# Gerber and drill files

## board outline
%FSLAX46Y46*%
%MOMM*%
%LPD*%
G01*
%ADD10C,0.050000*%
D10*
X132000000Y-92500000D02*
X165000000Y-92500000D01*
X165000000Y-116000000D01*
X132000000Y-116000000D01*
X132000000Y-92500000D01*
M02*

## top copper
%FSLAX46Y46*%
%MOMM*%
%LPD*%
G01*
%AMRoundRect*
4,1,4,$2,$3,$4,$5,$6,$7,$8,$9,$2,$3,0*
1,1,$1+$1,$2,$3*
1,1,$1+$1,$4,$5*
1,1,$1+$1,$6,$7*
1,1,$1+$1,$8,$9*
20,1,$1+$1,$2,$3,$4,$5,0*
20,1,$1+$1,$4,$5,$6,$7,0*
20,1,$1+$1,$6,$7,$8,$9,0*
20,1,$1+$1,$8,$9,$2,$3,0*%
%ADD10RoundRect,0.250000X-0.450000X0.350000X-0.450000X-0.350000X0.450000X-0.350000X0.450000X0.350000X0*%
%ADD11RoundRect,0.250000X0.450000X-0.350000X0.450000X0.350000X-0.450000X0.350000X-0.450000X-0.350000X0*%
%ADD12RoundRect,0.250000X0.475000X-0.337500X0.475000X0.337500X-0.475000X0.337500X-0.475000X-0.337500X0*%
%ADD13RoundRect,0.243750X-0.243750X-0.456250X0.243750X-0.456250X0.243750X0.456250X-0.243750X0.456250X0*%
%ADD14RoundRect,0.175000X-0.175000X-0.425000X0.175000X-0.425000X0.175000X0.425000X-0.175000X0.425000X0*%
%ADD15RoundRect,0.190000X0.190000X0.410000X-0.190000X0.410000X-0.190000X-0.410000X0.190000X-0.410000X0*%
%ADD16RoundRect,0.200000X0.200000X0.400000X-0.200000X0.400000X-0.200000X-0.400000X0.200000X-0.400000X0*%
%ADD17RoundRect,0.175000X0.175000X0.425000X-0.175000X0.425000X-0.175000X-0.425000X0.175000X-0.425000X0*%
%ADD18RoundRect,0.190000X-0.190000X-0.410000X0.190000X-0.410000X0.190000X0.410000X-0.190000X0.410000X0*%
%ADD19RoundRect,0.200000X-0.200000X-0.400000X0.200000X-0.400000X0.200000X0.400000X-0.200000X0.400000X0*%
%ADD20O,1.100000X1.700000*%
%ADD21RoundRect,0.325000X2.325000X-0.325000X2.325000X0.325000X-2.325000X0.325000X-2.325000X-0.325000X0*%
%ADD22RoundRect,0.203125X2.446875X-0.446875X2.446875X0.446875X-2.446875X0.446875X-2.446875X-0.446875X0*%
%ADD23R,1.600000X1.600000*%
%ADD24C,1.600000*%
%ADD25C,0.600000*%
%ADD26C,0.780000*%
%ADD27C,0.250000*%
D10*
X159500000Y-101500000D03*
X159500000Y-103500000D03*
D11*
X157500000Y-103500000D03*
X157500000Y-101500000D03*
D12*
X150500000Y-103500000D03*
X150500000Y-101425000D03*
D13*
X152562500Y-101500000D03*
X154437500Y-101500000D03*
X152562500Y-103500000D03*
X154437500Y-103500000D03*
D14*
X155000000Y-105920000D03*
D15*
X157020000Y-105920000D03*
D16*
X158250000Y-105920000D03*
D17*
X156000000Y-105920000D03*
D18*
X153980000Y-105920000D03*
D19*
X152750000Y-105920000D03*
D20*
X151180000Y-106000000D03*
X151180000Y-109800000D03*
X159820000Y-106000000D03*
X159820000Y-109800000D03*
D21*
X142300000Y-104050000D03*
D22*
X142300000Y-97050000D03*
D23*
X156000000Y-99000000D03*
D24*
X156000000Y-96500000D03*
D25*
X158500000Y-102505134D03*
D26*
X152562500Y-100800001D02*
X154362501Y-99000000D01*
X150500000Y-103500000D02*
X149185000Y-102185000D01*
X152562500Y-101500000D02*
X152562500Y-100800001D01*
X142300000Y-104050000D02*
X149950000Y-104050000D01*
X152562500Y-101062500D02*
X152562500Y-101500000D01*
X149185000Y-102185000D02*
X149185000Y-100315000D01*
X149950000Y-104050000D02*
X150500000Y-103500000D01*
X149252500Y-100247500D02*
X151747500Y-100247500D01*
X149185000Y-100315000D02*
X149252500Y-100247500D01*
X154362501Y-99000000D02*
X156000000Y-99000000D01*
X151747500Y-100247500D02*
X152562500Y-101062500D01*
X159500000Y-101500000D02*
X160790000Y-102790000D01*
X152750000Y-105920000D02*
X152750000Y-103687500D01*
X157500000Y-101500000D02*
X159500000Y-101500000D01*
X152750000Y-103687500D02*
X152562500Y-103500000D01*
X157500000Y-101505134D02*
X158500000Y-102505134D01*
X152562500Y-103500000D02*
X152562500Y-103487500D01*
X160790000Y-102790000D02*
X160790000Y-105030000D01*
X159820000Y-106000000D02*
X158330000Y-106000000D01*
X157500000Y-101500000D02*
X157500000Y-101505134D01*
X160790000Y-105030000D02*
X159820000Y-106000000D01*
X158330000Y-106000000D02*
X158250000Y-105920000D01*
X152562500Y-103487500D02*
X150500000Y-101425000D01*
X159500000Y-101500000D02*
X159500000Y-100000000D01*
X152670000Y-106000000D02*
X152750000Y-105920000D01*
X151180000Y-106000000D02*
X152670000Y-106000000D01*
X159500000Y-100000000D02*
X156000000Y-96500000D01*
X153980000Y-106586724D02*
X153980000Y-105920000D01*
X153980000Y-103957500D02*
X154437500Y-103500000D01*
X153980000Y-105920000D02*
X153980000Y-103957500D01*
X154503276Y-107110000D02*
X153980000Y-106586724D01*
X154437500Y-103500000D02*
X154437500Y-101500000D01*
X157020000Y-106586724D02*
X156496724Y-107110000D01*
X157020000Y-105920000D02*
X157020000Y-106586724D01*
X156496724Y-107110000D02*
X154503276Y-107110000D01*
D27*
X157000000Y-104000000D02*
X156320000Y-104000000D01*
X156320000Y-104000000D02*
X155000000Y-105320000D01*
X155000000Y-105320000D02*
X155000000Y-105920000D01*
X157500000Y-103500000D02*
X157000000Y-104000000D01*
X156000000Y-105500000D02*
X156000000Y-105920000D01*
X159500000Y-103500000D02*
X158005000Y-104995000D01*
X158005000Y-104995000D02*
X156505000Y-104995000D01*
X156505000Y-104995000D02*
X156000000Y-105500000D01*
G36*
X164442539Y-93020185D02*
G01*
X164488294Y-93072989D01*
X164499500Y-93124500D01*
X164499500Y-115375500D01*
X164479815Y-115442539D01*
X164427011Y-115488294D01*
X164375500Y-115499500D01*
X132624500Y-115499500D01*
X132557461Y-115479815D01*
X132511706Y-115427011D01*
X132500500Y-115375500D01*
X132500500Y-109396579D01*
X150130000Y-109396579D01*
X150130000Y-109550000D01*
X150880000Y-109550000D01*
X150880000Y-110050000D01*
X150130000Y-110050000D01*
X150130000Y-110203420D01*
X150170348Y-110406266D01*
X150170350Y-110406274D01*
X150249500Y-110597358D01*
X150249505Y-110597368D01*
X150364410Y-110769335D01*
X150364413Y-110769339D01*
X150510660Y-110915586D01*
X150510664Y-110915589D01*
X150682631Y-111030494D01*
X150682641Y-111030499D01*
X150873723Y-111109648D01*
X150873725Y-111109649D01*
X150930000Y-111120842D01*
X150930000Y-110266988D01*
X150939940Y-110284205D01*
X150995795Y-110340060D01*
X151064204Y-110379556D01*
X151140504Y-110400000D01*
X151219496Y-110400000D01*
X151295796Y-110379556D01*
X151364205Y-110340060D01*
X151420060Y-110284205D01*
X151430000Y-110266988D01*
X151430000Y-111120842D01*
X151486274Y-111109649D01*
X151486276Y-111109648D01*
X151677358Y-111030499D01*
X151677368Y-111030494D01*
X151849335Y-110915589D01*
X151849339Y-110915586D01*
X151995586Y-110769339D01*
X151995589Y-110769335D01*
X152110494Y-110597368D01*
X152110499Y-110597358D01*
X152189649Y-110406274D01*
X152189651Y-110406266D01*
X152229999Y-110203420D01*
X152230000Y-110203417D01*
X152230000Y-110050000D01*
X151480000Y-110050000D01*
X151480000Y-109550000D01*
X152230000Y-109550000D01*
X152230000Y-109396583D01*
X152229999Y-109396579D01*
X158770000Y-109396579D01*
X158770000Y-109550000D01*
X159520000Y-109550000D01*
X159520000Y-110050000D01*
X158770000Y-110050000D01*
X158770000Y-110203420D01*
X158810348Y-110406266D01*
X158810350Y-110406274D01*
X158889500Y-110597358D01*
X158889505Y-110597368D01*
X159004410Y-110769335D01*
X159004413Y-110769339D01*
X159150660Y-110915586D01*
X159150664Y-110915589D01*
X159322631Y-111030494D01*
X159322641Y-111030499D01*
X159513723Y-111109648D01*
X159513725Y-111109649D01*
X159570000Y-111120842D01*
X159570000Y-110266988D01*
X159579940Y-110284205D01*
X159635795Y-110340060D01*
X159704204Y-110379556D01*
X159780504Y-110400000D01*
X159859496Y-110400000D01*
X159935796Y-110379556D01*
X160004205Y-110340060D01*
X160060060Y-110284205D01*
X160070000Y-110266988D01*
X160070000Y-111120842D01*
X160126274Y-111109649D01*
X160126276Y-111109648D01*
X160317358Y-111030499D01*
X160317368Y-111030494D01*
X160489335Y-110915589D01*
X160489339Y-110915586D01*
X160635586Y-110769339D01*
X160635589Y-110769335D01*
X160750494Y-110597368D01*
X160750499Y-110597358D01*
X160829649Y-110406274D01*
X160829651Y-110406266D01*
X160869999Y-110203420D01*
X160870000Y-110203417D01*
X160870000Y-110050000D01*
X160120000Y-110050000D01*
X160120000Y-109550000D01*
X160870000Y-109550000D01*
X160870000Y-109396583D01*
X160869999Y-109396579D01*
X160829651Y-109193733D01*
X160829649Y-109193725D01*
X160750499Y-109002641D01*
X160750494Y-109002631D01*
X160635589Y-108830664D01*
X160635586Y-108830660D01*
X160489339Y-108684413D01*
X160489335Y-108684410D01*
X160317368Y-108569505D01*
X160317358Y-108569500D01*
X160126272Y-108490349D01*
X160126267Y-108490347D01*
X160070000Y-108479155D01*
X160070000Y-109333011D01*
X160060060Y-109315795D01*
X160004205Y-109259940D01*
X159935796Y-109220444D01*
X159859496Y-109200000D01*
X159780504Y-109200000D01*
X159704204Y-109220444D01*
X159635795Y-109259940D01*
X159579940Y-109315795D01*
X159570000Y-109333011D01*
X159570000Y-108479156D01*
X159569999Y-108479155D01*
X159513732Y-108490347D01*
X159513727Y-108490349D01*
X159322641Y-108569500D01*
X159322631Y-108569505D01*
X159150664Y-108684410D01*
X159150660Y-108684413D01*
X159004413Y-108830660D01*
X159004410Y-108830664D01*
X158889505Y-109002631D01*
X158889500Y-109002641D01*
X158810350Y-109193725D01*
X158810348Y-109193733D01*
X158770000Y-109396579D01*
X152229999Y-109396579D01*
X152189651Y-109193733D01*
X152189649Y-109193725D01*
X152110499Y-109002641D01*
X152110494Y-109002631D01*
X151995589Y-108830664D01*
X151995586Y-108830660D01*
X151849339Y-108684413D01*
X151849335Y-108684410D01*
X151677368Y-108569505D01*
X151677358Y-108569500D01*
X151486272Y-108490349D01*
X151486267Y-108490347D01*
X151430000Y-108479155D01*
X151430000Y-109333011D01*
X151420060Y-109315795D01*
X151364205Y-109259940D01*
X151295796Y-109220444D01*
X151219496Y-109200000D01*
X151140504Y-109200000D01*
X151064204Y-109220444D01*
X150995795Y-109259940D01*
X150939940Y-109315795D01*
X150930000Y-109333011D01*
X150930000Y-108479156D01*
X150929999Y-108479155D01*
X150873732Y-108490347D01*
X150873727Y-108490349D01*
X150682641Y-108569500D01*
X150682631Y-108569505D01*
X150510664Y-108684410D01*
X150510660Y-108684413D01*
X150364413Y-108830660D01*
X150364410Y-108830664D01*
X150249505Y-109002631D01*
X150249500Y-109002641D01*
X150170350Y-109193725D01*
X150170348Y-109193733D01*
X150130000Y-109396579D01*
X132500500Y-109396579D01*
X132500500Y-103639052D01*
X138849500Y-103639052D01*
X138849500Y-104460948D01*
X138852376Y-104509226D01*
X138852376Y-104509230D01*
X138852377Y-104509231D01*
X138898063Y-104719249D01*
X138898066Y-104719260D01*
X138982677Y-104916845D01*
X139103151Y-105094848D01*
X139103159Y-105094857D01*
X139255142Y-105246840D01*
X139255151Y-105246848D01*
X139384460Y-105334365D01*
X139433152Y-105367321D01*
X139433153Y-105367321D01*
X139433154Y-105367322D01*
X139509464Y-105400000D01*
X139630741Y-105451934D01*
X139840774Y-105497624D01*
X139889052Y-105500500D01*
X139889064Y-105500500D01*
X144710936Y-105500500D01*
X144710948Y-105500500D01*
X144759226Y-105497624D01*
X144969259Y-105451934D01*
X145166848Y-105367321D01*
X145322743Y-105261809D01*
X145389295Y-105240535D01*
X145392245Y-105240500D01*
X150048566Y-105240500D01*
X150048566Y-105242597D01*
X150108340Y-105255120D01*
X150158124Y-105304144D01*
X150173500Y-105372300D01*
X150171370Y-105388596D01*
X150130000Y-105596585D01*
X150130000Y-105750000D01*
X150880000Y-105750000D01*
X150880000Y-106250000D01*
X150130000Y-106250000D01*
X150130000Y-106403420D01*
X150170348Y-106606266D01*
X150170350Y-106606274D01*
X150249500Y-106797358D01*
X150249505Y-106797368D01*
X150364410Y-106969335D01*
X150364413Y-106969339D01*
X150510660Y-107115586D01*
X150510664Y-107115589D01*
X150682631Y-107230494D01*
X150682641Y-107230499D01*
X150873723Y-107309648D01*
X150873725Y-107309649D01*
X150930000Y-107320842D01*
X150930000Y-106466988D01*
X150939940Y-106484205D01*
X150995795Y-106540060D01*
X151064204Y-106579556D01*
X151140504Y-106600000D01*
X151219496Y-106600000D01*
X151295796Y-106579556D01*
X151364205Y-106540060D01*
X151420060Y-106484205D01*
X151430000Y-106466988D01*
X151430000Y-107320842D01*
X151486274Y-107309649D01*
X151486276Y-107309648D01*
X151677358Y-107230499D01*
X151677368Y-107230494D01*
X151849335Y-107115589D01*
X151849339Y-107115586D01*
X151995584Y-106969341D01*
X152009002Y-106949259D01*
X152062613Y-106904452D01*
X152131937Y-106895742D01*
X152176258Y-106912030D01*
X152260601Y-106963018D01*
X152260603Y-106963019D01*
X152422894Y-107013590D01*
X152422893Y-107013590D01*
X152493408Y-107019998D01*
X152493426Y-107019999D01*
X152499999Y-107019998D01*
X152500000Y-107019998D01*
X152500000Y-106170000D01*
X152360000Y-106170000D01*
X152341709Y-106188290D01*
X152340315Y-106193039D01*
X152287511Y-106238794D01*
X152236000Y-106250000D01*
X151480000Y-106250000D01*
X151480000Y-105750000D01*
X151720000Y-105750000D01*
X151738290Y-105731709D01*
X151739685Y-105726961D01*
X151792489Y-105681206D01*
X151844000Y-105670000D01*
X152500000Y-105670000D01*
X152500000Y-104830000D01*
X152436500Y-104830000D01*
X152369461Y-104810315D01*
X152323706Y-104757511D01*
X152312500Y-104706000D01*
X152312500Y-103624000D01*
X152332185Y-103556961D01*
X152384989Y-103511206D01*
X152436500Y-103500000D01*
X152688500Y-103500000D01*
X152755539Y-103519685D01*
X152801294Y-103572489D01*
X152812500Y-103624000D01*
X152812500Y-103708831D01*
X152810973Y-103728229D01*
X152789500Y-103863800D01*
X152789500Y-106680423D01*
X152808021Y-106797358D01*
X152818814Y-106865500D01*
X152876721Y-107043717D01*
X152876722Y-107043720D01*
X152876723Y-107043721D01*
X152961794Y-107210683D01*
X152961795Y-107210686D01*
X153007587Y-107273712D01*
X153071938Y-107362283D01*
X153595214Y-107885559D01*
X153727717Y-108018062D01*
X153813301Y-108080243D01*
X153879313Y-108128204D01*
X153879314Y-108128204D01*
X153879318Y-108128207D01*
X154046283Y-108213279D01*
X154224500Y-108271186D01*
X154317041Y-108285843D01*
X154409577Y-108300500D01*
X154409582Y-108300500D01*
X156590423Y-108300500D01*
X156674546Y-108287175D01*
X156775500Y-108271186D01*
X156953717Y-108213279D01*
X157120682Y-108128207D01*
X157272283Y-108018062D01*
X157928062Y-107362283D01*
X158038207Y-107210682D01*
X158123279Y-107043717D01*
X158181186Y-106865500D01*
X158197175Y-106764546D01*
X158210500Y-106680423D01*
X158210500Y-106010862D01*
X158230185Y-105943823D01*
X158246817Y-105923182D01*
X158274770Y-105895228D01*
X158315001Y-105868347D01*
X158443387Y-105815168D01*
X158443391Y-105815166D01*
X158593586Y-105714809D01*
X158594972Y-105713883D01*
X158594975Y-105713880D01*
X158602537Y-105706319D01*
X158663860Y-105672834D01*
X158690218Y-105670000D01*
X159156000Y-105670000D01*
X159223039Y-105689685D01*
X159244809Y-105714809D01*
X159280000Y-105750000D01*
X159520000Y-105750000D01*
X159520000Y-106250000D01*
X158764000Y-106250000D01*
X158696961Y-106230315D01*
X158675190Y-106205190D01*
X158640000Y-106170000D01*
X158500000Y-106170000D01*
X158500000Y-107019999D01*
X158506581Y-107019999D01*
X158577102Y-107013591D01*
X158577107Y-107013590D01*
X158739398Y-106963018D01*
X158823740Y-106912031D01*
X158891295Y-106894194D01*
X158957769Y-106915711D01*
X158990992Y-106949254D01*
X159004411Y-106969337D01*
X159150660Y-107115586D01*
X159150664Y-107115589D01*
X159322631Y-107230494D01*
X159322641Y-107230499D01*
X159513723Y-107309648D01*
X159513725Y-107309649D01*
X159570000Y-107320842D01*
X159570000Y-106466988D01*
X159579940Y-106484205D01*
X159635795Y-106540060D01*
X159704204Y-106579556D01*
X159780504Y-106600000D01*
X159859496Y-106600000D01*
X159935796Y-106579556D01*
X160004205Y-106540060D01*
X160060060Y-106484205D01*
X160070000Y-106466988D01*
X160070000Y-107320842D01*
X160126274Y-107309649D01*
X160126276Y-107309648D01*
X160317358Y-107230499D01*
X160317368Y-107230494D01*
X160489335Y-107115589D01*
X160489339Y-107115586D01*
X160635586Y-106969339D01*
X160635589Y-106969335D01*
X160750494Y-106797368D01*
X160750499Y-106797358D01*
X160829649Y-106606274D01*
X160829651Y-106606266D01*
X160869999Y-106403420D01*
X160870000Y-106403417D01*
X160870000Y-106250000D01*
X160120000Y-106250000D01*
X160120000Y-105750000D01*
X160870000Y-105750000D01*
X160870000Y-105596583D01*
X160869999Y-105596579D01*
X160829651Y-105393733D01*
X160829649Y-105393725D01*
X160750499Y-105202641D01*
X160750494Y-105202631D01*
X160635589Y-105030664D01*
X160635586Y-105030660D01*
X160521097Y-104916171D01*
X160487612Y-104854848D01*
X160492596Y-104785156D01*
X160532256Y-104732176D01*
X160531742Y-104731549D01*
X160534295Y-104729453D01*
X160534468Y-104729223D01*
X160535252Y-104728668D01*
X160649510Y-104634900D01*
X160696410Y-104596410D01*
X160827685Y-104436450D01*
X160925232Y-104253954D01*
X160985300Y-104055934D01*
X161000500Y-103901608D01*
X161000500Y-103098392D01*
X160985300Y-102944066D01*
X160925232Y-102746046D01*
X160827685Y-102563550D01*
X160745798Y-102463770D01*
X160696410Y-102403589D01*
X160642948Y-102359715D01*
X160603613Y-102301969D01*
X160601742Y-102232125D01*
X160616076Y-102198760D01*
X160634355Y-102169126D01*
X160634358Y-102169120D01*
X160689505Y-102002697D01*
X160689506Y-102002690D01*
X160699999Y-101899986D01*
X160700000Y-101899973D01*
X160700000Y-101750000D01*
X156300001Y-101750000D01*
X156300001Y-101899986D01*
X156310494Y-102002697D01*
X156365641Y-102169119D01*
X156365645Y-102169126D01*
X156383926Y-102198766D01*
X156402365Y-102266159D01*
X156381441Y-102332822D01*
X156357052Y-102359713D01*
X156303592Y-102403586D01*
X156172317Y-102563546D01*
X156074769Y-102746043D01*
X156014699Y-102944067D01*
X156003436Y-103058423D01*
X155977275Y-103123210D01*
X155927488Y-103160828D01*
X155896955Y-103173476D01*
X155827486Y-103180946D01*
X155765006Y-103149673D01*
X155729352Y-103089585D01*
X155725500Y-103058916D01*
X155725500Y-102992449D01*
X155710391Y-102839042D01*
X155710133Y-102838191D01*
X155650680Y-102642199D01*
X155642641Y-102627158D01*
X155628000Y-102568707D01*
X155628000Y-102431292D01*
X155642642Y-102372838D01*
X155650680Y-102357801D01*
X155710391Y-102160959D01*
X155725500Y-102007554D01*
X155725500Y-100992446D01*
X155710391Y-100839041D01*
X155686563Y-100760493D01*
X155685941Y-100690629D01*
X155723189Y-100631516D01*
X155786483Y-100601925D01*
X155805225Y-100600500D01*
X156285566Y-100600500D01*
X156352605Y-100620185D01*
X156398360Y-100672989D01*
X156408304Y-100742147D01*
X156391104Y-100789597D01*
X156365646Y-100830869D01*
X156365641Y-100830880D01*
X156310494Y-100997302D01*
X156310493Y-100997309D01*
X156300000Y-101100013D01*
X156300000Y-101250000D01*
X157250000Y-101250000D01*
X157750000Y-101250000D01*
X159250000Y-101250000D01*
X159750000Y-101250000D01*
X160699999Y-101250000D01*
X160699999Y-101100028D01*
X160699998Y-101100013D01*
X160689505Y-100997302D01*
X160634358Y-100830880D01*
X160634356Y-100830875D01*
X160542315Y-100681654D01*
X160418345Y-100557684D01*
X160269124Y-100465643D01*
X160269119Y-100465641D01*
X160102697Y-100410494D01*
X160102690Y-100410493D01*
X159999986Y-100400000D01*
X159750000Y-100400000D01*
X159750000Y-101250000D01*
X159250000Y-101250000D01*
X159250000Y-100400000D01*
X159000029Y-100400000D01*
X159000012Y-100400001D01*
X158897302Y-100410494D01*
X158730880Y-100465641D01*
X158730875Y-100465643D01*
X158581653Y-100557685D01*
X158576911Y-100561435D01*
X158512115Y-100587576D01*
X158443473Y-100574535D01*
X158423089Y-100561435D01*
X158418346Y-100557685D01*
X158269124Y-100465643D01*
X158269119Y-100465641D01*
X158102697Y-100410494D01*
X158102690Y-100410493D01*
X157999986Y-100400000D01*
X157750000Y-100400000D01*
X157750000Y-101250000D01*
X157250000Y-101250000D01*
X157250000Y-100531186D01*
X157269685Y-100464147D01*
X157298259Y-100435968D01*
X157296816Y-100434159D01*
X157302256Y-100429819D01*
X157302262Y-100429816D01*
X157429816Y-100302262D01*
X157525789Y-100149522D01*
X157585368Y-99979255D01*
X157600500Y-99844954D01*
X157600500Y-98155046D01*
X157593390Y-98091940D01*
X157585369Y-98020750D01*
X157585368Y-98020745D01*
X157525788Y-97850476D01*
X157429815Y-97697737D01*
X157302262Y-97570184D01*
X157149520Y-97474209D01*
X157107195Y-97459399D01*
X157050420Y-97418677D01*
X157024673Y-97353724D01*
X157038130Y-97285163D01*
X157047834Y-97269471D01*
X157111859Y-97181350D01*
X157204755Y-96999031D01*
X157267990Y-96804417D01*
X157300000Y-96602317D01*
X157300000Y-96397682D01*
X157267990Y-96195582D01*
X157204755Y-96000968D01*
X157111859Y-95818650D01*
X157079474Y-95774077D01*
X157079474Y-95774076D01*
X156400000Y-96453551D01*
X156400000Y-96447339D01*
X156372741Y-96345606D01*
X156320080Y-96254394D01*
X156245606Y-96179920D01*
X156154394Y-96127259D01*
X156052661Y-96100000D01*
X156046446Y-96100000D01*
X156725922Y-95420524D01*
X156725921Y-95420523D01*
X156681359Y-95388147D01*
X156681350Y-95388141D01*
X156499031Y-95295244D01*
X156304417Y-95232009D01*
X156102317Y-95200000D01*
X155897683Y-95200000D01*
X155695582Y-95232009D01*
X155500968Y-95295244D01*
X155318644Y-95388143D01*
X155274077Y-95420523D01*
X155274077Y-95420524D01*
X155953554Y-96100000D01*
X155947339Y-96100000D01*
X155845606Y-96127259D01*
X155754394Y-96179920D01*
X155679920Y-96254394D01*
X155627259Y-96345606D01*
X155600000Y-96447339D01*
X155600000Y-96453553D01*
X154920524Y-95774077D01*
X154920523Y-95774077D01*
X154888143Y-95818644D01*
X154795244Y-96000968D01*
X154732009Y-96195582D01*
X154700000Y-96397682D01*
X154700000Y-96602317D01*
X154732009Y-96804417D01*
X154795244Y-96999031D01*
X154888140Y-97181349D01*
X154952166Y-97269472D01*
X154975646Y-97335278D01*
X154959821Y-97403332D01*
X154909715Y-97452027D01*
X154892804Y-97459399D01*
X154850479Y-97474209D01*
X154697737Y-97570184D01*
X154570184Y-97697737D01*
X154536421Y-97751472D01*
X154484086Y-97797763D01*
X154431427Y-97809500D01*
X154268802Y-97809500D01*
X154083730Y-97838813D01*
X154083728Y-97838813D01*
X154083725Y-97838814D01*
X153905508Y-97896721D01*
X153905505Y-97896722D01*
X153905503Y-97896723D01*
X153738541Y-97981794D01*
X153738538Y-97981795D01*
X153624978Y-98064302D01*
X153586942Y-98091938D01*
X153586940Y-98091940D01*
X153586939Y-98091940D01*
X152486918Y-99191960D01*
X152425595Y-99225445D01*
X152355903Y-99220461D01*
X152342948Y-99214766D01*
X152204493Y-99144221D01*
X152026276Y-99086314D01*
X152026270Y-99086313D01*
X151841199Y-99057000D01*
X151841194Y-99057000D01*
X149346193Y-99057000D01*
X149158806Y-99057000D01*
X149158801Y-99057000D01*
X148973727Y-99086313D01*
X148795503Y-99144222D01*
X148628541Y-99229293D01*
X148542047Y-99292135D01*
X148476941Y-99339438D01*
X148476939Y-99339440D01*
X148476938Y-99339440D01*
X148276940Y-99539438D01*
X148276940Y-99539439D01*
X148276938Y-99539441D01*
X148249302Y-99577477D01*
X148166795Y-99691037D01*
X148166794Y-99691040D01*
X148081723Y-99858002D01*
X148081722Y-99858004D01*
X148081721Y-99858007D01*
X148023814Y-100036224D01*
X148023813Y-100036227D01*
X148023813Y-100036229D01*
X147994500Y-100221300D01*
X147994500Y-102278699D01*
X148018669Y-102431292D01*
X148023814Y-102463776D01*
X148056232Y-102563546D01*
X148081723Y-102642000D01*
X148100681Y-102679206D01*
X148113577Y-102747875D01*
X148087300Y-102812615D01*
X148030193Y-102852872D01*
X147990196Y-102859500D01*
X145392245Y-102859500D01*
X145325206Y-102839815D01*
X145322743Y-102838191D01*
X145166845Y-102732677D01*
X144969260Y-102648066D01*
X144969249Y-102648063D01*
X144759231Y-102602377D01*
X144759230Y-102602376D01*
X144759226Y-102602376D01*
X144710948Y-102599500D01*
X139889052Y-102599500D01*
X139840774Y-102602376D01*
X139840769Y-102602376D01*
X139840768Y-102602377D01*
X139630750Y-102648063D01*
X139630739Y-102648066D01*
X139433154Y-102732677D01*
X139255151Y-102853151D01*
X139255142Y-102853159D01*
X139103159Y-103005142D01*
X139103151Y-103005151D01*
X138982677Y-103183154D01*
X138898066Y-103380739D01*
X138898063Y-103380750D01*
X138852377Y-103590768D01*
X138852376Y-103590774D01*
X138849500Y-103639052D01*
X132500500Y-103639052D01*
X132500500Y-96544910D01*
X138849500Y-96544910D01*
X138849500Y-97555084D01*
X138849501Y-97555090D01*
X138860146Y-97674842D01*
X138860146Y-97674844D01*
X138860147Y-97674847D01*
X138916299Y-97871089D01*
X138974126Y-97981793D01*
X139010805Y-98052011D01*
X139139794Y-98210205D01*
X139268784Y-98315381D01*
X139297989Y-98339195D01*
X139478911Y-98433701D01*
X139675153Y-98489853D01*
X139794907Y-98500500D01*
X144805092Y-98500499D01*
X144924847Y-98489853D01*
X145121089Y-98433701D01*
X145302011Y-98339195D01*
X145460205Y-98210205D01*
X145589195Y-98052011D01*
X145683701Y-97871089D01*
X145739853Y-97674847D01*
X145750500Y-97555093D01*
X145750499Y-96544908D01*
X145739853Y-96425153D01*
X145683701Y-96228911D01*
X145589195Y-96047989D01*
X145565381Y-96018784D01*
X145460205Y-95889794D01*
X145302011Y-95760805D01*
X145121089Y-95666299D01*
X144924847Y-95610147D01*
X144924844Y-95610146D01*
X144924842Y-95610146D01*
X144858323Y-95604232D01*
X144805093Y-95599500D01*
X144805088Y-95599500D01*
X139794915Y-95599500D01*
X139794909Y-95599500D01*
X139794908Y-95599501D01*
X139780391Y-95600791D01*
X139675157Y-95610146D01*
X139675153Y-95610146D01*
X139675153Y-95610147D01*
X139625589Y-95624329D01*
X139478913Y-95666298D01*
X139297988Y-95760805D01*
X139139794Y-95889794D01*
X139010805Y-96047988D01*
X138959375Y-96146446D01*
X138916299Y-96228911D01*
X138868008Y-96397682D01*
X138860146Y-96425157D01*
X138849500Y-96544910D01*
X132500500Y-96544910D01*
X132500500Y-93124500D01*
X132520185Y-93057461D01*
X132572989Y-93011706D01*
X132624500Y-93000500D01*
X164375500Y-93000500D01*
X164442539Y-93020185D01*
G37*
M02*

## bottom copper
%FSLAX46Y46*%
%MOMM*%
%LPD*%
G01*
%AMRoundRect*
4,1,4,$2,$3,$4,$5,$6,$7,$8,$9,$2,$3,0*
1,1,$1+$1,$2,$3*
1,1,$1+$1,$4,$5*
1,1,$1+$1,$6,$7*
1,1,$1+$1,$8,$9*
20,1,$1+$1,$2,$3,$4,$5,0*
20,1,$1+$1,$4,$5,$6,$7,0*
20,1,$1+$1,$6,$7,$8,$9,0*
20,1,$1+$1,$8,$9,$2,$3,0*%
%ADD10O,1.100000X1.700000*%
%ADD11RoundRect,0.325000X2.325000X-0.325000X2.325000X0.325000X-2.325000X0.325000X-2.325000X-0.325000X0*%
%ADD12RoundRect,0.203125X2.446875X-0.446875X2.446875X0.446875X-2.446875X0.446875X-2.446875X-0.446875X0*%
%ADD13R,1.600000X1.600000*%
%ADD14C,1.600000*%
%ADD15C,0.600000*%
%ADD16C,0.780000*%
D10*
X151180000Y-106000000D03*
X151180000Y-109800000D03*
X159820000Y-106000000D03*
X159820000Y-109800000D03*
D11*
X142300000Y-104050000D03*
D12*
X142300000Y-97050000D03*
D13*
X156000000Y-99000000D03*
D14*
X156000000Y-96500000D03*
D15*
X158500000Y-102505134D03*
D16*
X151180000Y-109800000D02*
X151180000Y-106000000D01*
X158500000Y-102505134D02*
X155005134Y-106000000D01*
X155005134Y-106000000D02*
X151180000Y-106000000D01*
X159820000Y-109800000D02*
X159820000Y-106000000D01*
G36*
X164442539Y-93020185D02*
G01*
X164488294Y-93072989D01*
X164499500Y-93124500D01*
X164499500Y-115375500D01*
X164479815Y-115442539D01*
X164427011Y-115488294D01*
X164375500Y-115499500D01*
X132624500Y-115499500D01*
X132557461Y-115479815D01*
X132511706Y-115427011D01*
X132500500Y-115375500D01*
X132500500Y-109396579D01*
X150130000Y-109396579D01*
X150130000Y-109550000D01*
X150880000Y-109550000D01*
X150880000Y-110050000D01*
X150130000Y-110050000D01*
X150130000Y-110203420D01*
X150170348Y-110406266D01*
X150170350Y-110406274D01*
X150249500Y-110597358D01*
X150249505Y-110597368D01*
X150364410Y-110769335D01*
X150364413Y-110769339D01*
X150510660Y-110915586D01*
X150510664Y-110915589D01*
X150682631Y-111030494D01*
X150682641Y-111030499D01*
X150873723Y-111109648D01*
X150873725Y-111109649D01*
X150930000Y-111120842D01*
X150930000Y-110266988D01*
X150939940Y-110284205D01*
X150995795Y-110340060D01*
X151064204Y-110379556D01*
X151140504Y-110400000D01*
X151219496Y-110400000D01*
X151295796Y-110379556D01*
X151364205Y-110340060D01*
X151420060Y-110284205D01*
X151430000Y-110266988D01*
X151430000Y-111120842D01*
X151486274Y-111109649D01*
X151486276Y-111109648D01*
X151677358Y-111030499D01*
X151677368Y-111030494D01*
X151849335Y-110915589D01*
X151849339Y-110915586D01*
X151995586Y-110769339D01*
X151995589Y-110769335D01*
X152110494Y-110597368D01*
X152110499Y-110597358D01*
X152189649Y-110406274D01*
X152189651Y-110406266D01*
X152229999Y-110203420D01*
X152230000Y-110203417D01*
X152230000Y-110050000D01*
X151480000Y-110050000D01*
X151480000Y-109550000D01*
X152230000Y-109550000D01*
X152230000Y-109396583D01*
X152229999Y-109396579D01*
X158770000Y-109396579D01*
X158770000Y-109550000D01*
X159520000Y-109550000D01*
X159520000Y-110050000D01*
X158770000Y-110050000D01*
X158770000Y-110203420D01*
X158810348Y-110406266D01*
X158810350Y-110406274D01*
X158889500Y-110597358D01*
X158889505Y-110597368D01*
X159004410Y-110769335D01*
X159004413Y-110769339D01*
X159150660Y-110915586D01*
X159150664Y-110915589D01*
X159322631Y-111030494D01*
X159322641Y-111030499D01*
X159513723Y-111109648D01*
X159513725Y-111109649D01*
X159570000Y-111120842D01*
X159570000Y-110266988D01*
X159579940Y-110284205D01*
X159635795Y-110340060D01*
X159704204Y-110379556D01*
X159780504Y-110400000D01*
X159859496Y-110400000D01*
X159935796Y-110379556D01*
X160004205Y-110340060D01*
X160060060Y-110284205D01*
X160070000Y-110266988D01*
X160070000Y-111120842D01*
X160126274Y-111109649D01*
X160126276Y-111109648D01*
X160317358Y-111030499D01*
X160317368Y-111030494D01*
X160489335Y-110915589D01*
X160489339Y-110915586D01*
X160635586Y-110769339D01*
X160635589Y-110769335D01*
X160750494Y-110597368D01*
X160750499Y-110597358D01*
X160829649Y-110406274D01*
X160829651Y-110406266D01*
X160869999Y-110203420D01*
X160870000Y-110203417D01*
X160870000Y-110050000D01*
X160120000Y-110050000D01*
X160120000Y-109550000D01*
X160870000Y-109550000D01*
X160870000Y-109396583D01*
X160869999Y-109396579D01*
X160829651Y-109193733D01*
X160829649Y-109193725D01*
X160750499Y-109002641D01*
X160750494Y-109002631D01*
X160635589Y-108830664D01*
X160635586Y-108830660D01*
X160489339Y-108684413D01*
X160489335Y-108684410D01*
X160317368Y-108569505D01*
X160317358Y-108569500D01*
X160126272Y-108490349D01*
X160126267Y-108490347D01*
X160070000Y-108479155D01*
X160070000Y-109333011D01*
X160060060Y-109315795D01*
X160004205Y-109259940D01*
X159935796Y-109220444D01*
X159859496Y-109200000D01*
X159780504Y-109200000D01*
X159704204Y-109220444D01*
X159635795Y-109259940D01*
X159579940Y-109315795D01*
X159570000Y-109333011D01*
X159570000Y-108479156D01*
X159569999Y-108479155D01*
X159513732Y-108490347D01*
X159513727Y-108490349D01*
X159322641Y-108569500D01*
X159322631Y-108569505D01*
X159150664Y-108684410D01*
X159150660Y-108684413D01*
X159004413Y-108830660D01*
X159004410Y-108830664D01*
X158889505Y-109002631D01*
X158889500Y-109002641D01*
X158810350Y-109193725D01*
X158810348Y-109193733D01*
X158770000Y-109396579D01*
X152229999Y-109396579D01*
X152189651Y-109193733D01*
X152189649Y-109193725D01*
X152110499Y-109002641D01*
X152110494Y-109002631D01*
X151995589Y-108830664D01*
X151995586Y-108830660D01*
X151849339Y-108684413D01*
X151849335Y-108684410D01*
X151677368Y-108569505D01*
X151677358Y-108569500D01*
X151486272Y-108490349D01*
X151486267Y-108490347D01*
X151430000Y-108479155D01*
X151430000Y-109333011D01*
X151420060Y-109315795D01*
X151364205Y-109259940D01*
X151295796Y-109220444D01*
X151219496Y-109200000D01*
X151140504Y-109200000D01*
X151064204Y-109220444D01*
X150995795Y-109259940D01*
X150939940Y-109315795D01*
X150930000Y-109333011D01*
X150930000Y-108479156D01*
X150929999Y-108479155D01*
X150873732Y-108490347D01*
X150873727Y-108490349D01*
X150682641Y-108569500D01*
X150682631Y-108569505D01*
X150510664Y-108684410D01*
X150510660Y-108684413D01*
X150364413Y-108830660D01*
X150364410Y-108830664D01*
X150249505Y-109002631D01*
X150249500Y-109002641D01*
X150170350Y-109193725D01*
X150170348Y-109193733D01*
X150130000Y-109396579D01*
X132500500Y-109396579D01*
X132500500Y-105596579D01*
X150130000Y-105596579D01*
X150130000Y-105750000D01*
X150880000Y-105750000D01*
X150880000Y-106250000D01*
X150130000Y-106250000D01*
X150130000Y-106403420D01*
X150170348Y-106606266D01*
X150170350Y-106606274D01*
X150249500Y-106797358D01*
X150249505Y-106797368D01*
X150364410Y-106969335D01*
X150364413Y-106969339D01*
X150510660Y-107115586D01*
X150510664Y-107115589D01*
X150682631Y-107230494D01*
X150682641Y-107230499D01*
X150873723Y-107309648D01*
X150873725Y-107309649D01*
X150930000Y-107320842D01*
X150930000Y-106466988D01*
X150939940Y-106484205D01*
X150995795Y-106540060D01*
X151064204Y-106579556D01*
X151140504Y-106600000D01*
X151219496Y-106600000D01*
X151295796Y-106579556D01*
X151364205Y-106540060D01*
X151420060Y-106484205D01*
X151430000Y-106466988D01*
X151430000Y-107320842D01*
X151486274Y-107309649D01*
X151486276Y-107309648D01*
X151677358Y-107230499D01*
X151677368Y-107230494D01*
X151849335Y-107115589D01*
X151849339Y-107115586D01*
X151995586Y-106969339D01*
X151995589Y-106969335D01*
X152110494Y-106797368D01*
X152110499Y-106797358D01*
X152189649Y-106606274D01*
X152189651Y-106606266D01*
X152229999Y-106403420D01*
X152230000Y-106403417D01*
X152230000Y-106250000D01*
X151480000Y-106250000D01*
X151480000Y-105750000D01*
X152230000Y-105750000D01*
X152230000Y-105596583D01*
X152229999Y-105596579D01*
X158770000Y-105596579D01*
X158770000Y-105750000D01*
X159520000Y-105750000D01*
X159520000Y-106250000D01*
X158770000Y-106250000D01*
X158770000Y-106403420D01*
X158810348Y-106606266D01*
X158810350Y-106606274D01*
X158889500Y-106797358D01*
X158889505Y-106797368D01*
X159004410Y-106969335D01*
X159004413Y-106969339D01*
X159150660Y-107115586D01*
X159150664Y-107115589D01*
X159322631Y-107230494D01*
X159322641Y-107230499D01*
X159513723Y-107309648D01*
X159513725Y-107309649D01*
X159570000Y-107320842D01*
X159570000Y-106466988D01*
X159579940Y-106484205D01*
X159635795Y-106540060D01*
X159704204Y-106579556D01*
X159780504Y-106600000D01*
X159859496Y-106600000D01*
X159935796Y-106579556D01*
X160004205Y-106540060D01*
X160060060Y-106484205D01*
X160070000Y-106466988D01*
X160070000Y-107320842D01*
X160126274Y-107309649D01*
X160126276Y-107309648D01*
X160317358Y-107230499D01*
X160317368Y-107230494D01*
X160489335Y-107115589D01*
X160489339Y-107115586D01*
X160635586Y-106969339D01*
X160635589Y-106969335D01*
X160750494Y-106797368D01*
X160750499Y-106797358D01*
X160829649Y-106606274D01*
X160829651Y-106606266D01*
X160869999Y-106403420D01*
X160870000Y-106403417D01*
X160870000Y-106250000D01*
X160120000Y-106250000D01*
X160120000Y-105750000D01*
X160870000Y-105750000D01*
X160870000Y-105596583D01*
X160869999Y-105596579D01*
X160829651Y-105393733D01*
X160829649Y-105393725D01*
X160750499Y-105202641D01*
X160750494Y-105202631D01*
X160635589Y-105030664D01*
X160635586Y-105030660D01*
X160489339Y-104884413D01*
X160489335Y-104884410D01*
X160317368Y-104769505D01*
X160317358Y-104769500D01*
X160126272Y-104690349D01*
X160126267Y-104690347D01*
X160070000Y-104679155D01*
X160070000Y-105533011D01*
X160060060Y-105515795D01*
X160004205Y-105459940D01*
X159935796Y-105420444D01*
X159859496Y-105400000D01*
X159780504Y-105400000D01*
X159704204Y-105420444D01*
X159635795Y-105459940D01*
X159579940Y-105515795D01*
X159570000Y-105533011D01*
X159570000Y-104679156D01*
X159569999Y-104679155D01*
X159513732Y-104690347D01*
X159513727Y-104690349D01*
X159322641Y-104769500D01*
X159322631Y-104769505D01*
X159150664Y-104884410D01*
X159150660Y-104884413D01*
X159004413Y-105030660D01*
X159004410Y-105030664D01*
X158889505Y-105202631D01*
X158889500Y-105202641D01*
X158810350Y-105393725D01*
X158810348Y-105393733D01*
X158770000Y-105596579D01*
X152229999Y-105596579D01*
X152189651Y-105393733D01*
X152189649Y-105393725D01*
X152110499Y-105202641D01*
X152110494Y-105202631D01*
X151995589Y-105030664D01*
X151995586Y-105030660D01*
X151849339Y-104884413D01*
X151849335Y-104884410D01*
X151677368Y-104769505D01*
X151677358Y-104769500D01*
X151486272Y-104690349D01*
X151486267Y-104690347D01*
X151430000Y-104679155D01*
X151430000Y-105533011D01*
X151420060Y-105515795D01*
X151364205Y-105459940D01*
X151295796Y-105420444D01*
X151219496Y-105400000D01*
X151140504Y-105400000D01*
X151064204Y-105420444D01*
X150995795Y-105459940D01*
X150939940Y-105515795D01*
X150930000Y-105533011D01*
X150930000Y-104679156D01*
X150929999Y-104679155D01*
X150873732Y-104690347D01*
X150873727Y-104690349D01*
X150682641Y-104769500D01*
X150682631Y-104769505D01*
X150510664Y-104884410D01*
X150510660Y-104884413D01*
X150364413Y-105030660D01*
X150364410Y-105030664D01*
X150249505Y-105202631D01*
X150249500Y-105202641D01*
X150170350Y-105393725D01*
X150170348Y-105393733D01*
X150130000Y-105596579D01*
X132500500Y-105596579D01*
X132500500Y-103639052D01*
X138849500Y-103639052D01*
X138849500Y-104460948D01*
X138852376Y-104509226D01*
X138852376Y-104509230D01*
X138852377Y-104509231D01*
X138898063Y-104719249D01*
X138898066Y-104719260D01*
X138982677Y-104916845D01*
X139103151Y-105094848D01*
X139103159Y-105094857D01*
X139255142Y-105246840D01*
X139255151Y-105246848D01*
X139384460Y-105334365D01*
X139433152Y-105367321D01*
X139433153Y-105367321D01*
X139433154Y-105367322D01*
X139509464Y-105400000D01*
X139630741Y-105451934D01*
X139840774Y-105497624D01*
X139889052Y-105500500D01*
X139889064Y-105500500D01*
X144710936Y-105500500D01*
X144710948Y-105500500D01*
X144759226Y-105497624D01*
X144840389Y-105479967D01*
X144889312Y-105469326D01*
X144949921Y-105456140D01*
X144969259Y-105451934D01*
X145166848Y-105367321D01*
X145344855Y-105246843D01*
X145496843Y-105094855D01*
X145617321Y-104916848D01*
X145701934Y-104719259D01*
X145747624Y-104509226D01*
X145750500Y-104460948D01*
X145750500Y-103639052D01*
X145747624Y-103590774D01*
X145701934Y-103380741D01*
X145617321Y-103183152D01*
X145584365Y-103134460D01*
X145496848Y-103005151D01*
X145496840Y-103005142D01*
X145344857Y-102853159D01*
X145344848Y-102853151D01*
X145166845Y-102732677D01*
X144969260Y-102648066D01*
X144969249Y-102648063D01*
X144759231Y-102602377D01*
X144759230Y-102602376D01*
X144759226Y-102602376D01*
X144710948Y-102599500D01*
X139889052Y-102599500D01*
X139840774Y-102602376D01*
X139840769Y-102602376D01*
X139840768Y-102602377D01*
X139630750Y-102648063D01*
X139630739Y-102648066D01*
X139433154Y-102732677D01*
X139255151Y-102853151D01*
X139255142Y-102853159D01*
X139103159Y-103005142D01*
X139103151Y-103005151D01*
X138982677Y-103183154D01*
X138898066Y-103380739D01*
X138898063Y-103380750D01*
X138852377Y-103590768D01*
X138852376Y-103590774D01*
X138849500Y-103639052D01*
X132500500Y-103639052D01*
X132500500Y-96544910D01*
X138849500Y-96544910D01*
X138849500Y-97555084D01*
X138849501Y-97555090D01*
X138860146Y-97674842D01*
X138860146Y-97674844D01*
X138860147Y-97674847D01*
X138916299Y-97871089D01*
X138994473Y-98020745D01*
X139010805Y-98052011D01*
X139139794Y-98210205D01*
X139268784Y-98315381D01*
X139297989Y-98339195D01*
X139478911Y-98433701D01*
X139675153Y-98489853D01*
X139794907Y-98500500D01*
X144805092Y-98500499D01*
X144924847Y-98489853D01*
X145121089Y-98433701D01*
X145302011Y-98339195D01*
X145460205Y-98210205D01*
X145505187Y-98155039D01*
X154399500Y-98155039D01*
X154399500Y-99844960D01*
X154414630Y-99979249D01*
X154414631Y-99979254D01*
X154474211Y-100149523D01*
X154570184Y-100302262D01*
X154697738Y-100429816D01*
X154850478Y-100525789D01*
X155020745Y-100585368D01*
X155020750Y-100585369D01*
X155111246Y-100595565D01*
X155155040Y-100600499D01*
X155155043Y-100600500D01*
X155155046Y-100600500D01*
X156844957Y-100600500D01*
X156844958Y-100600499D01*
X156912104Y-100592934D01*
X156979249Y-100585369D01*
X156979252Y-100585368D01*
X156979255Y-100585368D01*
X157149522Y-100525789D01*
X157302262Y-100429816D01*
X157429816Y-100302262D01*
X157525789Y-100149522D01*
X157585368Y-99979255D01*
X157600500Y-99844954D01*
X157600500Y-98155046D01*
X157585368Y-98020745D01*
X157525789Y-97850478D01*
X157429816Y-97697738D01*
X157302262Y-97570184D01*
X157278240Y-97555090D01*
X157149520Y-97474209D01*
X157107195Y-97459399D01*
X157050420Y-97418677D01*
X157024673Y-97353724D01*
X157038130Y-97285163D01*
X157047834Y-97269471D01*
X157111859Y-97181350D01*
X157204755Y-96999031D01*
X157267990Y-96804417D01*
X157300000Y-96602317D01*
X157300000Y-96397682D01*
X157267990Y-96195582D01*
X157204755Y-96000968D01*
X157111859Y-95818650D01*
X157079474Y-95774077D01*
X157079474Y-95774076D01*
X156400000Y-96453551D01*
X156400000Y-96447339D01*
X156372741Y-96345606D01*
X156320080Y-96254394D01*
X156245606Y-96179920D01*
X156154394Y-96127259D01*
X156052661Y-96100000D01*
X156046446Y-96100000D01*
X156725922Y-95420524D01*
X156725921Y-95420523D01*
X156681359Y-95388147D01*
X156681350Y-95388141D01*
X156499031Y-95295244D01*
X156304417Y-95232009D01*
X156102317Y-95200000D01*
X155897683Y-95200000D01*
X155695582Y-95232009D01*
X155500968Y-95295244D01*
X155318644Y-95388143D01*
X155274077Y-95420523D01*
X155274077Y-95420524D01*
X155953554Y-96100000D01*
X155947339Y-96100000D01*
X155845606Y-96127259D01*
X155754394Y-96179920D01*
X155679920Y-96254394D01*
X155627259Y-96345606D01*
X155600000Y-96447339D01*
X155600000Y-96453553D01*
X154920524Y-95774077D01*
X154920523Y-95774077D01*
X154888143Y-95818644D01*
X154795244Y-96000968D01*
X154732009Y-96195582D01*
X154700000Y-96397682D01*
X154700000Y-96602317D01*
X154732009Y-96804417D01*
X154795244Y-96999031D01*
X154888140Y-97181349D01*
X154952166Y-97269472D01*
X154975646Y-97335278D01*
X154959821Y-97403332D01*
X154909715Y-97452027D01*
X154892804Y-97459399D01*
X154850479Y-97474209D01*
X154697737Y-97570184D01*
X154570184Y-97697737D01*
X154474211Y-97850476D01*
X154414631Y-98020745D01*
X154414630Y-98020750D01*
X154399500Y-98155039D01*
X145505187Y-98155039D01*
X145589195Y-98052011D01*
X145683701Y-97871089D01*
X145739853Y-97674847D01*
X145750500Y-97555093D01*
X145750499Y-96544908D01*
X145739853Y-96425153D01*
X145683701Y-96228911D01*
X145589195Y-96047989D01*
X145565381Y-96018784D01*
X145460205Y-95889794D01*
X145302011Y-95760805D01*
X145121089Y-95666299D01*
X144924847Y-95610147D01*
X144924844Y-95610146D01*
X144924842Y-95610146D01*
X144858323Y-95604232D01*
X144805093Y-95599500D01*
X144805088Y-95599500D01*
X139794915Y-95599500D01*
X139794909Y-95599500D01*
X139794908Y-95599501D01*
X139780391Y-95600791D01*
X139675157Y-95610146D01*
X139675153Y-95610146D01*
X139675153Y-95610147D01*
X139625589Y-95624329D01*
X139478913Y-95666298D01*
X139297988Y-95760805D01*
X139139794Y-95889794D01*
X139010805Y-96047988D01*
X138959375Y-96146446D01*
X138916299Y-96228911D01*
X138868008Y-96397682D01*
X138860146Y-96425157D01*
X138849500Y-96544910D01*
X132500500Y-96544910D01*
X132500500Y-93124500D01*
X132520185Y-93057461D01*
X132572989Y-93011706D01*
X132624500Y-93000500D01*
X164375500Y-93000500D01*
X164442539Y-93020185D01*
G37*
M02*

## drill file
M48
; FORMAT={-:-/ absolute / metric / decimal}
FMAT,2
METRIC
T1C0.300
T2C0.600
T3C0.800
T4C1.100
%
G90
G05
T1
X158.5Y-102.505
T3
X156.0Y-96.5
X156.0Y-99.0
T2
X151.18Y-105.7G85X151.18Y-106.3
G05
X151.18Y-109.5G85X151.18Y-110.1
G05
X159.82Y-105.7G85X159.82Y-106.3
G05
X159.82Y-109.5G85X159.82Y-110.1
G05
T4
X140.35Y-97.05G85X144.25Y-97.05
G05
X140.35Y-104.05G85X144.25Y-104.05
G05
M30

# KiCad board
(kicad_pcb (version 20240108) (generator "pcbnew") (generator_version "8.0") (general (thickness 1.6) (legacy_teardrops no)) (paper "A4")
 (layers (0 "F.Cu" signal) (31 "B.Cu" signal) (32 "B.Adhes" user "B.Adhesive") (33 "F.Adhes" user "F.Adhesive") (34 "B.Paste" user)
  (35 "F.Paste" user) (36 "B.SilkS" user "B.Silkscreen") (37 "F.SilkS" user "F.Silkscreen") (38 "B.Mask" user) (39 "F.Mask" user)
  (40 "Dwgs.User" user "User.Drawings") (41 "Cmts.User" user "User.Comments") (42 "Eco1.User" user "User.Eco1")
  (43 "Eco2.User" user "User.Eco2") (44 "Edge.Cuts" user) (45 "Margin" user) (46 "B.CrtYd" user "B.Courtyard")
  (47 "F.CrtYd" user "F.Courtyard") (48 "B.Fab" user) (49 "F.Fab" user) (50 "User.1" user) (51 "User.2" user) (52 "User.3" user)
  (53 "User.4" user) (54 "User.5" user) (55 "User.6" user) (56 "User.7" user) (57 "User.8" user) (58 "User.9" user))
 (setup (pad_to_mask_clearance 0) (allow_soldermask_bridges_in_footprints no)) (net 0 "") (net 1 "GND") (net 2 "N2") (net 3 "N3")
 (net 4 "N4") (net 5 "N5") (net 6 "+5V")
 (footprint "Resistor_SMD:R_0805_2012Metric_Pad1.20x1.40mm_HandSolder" (layer "F.Cu") (at 159.5 102.5 -90)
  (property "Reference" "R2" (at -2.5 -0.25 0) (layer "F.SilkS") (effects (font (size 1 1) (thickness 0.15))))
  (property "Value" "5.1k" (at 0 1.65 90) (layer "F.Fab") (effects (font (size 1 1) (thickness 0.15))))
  (pad "1" smd roundrect (at -1 0 270) (size 1.2 1.4) (layers "F.Cu" "F.Paste" "F.Mask") (roundrect_rratio 0.208333) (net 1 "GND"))
  (pad "2" smd roundrect (at 1 0 270) (size 1.2 1.4) (layers "F.Cu" "F.Paste" "F.Mask") (roundrect_rratio 0.208333) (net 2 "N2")))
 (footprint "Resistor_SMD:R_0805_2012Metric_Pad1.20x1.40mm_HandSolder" (layer "F.Cu") (at 157.5 102.5 90)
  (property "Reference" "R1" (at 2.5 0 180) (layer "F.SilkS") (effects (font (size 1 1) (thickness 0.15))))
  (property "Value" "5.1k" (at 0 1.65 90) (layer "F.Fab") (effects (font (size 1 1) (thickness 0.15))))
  (pad "1" smd roundrect (at -1 0 90) (size 1.2 1.4) (layers "F.Cu" "F.Paste" "F.Mask") (roundrect_rratio 0.208333) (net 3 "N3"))
  (pad "2" smd roundrect (at 1 0 90) (size 1.2 1.4) (layers "F.Cu" "F.Paste" "F.Mask") (roundrect_rratio 0.208333) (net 1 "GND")))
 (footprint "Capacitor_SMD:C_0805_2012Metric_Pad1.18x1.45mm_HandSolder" (layer "F.Cu") (at 150.5 102.4625 90)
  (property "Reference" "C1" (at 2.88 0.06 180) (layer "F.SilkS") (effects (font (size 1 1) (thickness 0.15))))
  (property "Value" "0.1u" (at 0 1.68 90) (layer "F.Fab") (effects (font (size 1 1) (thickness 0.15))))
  (pad "1" smd roundrect (at -1.0375 0 90) (size 1.175 1.45) (layers "F.Cu" "F.Paste" "F.Mask") (roundrect_rratio 0.212766) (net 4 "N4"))
  (pad "2" smd roundrect (at 1.0375 0 90) (size 1.175 1.45) (layers "F.Cu" "F.Paste" "F.Mask") (roundrect_rratio 0.212766) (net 1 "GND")))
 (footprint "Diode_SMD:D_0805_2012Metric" (layer "F.Cu") (at 153.5 101.5)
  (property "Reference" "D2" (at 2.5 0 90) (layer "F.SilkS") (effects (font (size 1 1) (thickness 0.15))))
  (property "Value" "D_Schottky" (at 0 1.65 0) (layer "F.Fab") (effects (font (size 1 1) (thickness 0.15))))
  (pad "1" smd roundrect (at -0.9375 0) (size 0.975 1.4) (layers "F.Cu" "F.Paste" "F.Mask") (roundrect_rratio 0.25) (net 4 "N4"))
  (pad "2" smd roundrect (at 0.9375 0) (size 0.975 1.4) (layers "F.Cu" "F.Paste" "F.Mask") (roundrect_rratio 0.25) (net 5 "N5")))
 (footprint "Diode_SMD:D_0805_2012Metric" (layer "F.Cu") (at 153.5 103.5)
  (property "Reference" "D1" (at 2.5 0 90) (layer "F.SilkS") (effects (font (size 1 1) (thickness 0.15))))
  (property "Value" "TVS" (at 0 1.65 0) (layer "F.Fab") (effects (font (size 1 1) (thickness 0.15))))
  (pad "1" smd roundrect (at -0.9375 0) (size 0.975 1.4) (layers "F.Cu" "F.Paste" "F.Mask") (roundrect_rratio 0.25) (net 1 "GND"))
  (pad "2" smd roundrect (at 0.9375 0) (size 0.975 1.4) (layers "F.Cu" "F.Paste" "F.Mask") (roundrect_rratio 0.25) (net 5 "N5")))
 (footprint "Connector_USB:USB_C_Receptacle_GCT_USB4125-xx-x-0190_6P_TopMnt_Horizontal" (layer "F.Cu") (at 155.5 109)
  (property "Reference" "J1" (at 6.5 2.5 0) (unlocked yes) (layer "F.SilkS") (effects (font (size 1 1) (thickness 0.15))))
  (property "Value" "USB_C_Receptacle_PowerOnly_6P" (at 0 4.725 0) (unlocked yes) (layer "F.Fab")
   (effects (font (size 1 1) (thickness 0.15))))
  (pad "A5" smd roundrect (at -0.5 -3.08) (size 0.7 1.2) (layers "F.Cu" "F.Paste" "F.Mask") (roundrect_rratio 0.25) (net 3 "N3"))
  (pad "A9" smd roundrect (at 1.52 -3.08 180) (size 0.76 1.2) (layers "F.Cu" "F.Paste" "F.Mask") (roundrect_rratio 0.25) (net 5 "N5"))
  (pad "A12" smd roundrect (at 2.75 -3.08 180) (size 0.8 1.2) (layers "F.Cu" "F.Paste" "F.Mask") (roundrect_rratio 0.25) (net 1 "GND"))
  (pad "B5" smd roundrect (at 0.5 -3.08 180) (size 0.7 1.2) (layers "F.Cu" "F.Paste" "F.Mask") (roundrect_rratio 0.25) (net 2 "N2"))
  (pad "B9" smd roundrect (at -1.52 -3.08) (size 0.76 1.2) (layers "F.Cu" "F.Paste" "F.Mask") (roundrect_rratio 0.25) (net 5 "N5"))
  (pad "B12" smd roundrect (at -2.75 -3.08) (size 0.8 1.2) (layers "F.Cu" "F.Paste" "F.Mask") (roundrect_rratio 0.25) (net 1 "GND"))
  (pad "S1" thru_hole oval (at -4.32 -3) (size 1.1 1.7) (drill oval 0.6 1.2) (layers "*.Cu" "*.Mask" "F.Paste") (remove_unused_layers no)
   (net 1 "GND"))
  (pad "S1" thru_hole oval (at -4.32 0.8) (size 1.1 1.7) (drill oval 0.6 1.2) (layers "*.Cu" "*.Mask" "F.Paste") (remove_unused_layers no)
   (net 1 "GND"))
  (pad "S1" thru_hole oval (at 4.32 -3) (size 1.1 1.7) (drill oval 0.6 1.2) (layers "*.Cu" "*.Mask" "F.Paste") (remove_unused_layers no)
   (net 1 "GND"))
  (pad "S1" thru_hole oval (at 4.32 0.8) (size 1.1 1.7) (drill oval 0.6 1.2) (layers "*.Cu" "*.Mask" "F.Paste") (remove_unused_layers no)
   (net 1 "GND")))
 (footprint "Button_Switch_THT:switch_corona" (layer "F.Cu") (at 142.3 104.05 90)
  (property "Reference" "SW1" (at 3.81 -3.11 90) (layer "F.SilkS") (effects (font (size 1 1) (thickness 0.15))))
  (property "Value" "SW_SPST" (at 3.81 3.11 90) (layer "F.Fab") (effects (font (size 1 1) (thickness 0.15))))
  (pad "1" thru_hole roundrect (at 0 0 90) (size 1.3 5.3) (drill oval 1.1 5) (layers "*.Cu" "*.Mask") (remove_unused_layers no)
   (roundrect_rratio 0.25) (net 4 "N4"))
  (pad "2" thru_hole roundrect (at 7 0 90) (size 1.3 5.3) (drill oval 1.1 5) (layers "*.Cu" "*.Mask") (remove_unused_layers no)
   (roundrect_rratio 0.15625) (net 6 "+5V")))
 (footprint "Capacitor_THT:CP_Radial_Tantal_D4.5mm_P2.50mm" (layer "F.Cu") (at 156 99 90)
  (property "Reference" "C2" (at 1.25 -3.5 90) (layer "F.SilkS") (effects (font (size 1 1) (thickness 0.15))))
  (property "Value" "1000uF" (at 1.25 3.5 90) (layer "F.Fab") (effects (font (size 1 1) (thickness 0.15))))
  (pad "1" thru_hole rect (at 0 0 90) (size 1.6 1.6) (drill 0.8) (layers "*.Cu" "*.Mask") (remove_unused_layers no) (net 4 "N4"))
  (pad "2" thru_hole circle (at 2.5 0 90) (size 1.6 1.6) (drill 0.8) (layers "*.Cu" "*.Mask") (remove_unused_layers no) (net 1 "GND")))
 (gr_rect (start 132 92.5) (end 165 116) (stroke (width 0.05) (type default)) (fill none) (layer "Edge.Cuts"))
 (segment (start 152.5625 100.800001) (end 154.362501 99) (width 0.78) (layer "F.Cu") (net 4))
 (segment (start 150.5 103.5) (end 149.185 102.185) (width 0.78) (layer "F.Cu") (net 4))
 (segment (start 152.5625 101.5) (end 152.5625 100.800001) (width 0.78) (layer "F.Cu") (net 4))
 (segment (start 142.3 104.05) (end 149.95 104.05) (width 0.78) (layer "F.Cu") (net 4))
 (segment (start 152.5625 101.0625) (end 152.5625 101.5) (width 0.78) (layer "F.Cu") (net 4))
 (segment (start 149.185 102.185) (end 149.185 100.315) (width 0.78) (layer "F.Cu") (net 4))
 (segment (start 149.95 104.05) (end 150.5 103.5) (width 0.78) (layer "F.Cu") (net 4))
 (segment (start 149.2525 100.2475) (end 151.7475 100.2475) (width 0.78) (layer "F.Cu") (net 4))
 (segment (start 149.185 100.315) (end 149.2525 100.2475) (width 0.78) (layer "F.Cu") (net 4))
 (segment (start 154.362501 99) (end 156 99) (width 0.78) (layer "F.Cu") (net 4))
 (segment (start 151.7475 100.2475) (end 152.5625 101.0625) (width 0.78) (layer "F.Cu") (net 4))
 (segment (start 159.5 101.5) (end 160.79 102.79) (width 0.78) (layer "F.Cu") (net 1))
 (segment (start 152.75 105.92) (end 152.75 103.6875) (width 0.78) (layer "F.Cu") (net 1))
 (segment (start 157.5 101.5) (end 159.5 101.5) (width 0.78) (layer "F.Cu") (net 1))
 (segment (start 152.75 103.6875) (end 152.5625 103.5) (width 0.78) (layer "F.Cu") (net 1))
 (segment (start 157.5 101.505134) (end 158.5 102.505134) (width 0.78) (layer "F.Cu") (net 1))
 (segment (start 152.5625 103.5) (end 152.5625 103.4875) (width 0.78) (layer "F.Cu") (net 1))
 (segment (start 160.79 102.79) (end 160.79 105.03) (width 0.78) (layer "F.Cu") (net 1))
 (segment (start 159.82 106) (end 158.33 106) (width 0.78) (layer "F.Cu") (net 1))
 (segment (start 157.5 101.5) (end 157.5 101.505134) (width 0.78) (layer "F.Cu") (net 1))
 (segment (start 160.79 105.03) (end 159.82 106) (width 0.78) (layer "F.Cu") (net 1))
 (segment (start 158.33 106) (end 158.25 105.92) (width 0.78) (layer "F.Cu") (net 1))
 (segment (start 152.5625 103.4875) (end 150.5 101.425) (width 0.78) (layer "F.Cu") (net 1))
 (segment (start 159.5 101.5) (end 159.5 100) (width 0.78) (layer "F.Cu") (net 1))
 (segment (start 152.67 106) (end 152.75 105.92) (width 0.78) (layer "F.Cu") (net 1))
 (segment (start 151.18 106) (end 152.67 106) (width 0.78) (layer "F.Cu") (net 1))
 (segment (start 159.5 100) (end 156 96.5) (width 0.78) (layer "F.Cu") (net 1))
 (via (at 158.5 102.505134) (size 0.6) (drill 0.3) (layers "F.Cu" "B.Cu") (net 1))
 (segment (start 151.18 109.8) (end 151.18 106) (width 0.78) (layer "B.Cu") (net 1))
 (segment (start 158.5 102.505134) (end 155.005134 106) (width 0.78) (layer "B.Cu") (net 1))
 (segment (start 155.005134 106) (end 151.18 106) (width 0.78) (layer "B.Cu") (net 1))
 (segment (start 159.82 109.8) (end 159.82 106) (width 0.78) (layer "B.Cu") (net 1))
 (segment (start 153.98 106.586724) (end 153.98 105.92) (width 0.78) (layer "F.Cu") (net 5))
 (segment (start 153.98 103.9575) (end 154.4375 103.5) (width 0.78) (layer "F.Cu") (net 5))
 (segment (start 153.98 105.92) (end 153.98 103.9575) (width 0.78) (layer "F.Cu") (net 5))
 (segment (start 154.503276 107.11) (end 153.98 106.586724) (width 0.78) (layer "F.Cu") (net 5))
 (segment (start 154.4375 103.5) (end 154.4375 101.5) (width 0.78) (layer "F.Cu") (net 5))
 (segment (start 157.02 106.586724) (end 156.496724 107.11) (width 0.78) (layer "F.Cu") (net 5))
 (segment (start 157.02 105.92) (end 157.02 106.586724) (width 0.78) (layer "F.Cu") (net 5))
 (segment (start 156.496724 107.11) (end 154.503276 107.11) (width 0.78) (layer "F.Cu") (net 5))
 (segment (start 157 104) (end 156.32 104) (width 0.25) (layer "F.Cu") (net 3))
 (segment (start 156.32 104) (end 155 105.32) (width 0.25) (layer "F.Cu") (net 3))
 (segment (start 155 105.32) (end 155 105.92) (width 0.25) (layer "F.Cu") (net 3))
 (segment (start 157.5 103.5) (end 157 104) (width 0.25) (layer "F.Cu") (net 3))
 (segment (start 156 105.5) (end 156 105.92) (width 0.25) (layer "F.Cu") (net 2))
 (segment (start 159.5 103.5) (end 158.005 104.995) (width 0.25) (layer "F.Cu") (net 2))
 (segment (start 158.005 104.995) (end 156.505 104.995) (width 0.25) (layer "F.Cu") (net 2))
 (segment (start 156.505 104.995) (end 156 105.5) (width 0.25) (layer "F.Cu") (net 2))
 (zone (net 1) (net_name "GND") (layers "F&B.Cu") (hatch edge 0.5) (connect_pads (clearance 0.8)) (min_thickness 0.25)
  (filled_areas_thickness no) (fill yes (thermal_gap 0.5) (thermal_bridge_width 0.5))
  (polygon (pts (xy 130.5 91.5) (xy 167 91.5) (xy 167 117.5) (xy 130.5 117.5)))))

